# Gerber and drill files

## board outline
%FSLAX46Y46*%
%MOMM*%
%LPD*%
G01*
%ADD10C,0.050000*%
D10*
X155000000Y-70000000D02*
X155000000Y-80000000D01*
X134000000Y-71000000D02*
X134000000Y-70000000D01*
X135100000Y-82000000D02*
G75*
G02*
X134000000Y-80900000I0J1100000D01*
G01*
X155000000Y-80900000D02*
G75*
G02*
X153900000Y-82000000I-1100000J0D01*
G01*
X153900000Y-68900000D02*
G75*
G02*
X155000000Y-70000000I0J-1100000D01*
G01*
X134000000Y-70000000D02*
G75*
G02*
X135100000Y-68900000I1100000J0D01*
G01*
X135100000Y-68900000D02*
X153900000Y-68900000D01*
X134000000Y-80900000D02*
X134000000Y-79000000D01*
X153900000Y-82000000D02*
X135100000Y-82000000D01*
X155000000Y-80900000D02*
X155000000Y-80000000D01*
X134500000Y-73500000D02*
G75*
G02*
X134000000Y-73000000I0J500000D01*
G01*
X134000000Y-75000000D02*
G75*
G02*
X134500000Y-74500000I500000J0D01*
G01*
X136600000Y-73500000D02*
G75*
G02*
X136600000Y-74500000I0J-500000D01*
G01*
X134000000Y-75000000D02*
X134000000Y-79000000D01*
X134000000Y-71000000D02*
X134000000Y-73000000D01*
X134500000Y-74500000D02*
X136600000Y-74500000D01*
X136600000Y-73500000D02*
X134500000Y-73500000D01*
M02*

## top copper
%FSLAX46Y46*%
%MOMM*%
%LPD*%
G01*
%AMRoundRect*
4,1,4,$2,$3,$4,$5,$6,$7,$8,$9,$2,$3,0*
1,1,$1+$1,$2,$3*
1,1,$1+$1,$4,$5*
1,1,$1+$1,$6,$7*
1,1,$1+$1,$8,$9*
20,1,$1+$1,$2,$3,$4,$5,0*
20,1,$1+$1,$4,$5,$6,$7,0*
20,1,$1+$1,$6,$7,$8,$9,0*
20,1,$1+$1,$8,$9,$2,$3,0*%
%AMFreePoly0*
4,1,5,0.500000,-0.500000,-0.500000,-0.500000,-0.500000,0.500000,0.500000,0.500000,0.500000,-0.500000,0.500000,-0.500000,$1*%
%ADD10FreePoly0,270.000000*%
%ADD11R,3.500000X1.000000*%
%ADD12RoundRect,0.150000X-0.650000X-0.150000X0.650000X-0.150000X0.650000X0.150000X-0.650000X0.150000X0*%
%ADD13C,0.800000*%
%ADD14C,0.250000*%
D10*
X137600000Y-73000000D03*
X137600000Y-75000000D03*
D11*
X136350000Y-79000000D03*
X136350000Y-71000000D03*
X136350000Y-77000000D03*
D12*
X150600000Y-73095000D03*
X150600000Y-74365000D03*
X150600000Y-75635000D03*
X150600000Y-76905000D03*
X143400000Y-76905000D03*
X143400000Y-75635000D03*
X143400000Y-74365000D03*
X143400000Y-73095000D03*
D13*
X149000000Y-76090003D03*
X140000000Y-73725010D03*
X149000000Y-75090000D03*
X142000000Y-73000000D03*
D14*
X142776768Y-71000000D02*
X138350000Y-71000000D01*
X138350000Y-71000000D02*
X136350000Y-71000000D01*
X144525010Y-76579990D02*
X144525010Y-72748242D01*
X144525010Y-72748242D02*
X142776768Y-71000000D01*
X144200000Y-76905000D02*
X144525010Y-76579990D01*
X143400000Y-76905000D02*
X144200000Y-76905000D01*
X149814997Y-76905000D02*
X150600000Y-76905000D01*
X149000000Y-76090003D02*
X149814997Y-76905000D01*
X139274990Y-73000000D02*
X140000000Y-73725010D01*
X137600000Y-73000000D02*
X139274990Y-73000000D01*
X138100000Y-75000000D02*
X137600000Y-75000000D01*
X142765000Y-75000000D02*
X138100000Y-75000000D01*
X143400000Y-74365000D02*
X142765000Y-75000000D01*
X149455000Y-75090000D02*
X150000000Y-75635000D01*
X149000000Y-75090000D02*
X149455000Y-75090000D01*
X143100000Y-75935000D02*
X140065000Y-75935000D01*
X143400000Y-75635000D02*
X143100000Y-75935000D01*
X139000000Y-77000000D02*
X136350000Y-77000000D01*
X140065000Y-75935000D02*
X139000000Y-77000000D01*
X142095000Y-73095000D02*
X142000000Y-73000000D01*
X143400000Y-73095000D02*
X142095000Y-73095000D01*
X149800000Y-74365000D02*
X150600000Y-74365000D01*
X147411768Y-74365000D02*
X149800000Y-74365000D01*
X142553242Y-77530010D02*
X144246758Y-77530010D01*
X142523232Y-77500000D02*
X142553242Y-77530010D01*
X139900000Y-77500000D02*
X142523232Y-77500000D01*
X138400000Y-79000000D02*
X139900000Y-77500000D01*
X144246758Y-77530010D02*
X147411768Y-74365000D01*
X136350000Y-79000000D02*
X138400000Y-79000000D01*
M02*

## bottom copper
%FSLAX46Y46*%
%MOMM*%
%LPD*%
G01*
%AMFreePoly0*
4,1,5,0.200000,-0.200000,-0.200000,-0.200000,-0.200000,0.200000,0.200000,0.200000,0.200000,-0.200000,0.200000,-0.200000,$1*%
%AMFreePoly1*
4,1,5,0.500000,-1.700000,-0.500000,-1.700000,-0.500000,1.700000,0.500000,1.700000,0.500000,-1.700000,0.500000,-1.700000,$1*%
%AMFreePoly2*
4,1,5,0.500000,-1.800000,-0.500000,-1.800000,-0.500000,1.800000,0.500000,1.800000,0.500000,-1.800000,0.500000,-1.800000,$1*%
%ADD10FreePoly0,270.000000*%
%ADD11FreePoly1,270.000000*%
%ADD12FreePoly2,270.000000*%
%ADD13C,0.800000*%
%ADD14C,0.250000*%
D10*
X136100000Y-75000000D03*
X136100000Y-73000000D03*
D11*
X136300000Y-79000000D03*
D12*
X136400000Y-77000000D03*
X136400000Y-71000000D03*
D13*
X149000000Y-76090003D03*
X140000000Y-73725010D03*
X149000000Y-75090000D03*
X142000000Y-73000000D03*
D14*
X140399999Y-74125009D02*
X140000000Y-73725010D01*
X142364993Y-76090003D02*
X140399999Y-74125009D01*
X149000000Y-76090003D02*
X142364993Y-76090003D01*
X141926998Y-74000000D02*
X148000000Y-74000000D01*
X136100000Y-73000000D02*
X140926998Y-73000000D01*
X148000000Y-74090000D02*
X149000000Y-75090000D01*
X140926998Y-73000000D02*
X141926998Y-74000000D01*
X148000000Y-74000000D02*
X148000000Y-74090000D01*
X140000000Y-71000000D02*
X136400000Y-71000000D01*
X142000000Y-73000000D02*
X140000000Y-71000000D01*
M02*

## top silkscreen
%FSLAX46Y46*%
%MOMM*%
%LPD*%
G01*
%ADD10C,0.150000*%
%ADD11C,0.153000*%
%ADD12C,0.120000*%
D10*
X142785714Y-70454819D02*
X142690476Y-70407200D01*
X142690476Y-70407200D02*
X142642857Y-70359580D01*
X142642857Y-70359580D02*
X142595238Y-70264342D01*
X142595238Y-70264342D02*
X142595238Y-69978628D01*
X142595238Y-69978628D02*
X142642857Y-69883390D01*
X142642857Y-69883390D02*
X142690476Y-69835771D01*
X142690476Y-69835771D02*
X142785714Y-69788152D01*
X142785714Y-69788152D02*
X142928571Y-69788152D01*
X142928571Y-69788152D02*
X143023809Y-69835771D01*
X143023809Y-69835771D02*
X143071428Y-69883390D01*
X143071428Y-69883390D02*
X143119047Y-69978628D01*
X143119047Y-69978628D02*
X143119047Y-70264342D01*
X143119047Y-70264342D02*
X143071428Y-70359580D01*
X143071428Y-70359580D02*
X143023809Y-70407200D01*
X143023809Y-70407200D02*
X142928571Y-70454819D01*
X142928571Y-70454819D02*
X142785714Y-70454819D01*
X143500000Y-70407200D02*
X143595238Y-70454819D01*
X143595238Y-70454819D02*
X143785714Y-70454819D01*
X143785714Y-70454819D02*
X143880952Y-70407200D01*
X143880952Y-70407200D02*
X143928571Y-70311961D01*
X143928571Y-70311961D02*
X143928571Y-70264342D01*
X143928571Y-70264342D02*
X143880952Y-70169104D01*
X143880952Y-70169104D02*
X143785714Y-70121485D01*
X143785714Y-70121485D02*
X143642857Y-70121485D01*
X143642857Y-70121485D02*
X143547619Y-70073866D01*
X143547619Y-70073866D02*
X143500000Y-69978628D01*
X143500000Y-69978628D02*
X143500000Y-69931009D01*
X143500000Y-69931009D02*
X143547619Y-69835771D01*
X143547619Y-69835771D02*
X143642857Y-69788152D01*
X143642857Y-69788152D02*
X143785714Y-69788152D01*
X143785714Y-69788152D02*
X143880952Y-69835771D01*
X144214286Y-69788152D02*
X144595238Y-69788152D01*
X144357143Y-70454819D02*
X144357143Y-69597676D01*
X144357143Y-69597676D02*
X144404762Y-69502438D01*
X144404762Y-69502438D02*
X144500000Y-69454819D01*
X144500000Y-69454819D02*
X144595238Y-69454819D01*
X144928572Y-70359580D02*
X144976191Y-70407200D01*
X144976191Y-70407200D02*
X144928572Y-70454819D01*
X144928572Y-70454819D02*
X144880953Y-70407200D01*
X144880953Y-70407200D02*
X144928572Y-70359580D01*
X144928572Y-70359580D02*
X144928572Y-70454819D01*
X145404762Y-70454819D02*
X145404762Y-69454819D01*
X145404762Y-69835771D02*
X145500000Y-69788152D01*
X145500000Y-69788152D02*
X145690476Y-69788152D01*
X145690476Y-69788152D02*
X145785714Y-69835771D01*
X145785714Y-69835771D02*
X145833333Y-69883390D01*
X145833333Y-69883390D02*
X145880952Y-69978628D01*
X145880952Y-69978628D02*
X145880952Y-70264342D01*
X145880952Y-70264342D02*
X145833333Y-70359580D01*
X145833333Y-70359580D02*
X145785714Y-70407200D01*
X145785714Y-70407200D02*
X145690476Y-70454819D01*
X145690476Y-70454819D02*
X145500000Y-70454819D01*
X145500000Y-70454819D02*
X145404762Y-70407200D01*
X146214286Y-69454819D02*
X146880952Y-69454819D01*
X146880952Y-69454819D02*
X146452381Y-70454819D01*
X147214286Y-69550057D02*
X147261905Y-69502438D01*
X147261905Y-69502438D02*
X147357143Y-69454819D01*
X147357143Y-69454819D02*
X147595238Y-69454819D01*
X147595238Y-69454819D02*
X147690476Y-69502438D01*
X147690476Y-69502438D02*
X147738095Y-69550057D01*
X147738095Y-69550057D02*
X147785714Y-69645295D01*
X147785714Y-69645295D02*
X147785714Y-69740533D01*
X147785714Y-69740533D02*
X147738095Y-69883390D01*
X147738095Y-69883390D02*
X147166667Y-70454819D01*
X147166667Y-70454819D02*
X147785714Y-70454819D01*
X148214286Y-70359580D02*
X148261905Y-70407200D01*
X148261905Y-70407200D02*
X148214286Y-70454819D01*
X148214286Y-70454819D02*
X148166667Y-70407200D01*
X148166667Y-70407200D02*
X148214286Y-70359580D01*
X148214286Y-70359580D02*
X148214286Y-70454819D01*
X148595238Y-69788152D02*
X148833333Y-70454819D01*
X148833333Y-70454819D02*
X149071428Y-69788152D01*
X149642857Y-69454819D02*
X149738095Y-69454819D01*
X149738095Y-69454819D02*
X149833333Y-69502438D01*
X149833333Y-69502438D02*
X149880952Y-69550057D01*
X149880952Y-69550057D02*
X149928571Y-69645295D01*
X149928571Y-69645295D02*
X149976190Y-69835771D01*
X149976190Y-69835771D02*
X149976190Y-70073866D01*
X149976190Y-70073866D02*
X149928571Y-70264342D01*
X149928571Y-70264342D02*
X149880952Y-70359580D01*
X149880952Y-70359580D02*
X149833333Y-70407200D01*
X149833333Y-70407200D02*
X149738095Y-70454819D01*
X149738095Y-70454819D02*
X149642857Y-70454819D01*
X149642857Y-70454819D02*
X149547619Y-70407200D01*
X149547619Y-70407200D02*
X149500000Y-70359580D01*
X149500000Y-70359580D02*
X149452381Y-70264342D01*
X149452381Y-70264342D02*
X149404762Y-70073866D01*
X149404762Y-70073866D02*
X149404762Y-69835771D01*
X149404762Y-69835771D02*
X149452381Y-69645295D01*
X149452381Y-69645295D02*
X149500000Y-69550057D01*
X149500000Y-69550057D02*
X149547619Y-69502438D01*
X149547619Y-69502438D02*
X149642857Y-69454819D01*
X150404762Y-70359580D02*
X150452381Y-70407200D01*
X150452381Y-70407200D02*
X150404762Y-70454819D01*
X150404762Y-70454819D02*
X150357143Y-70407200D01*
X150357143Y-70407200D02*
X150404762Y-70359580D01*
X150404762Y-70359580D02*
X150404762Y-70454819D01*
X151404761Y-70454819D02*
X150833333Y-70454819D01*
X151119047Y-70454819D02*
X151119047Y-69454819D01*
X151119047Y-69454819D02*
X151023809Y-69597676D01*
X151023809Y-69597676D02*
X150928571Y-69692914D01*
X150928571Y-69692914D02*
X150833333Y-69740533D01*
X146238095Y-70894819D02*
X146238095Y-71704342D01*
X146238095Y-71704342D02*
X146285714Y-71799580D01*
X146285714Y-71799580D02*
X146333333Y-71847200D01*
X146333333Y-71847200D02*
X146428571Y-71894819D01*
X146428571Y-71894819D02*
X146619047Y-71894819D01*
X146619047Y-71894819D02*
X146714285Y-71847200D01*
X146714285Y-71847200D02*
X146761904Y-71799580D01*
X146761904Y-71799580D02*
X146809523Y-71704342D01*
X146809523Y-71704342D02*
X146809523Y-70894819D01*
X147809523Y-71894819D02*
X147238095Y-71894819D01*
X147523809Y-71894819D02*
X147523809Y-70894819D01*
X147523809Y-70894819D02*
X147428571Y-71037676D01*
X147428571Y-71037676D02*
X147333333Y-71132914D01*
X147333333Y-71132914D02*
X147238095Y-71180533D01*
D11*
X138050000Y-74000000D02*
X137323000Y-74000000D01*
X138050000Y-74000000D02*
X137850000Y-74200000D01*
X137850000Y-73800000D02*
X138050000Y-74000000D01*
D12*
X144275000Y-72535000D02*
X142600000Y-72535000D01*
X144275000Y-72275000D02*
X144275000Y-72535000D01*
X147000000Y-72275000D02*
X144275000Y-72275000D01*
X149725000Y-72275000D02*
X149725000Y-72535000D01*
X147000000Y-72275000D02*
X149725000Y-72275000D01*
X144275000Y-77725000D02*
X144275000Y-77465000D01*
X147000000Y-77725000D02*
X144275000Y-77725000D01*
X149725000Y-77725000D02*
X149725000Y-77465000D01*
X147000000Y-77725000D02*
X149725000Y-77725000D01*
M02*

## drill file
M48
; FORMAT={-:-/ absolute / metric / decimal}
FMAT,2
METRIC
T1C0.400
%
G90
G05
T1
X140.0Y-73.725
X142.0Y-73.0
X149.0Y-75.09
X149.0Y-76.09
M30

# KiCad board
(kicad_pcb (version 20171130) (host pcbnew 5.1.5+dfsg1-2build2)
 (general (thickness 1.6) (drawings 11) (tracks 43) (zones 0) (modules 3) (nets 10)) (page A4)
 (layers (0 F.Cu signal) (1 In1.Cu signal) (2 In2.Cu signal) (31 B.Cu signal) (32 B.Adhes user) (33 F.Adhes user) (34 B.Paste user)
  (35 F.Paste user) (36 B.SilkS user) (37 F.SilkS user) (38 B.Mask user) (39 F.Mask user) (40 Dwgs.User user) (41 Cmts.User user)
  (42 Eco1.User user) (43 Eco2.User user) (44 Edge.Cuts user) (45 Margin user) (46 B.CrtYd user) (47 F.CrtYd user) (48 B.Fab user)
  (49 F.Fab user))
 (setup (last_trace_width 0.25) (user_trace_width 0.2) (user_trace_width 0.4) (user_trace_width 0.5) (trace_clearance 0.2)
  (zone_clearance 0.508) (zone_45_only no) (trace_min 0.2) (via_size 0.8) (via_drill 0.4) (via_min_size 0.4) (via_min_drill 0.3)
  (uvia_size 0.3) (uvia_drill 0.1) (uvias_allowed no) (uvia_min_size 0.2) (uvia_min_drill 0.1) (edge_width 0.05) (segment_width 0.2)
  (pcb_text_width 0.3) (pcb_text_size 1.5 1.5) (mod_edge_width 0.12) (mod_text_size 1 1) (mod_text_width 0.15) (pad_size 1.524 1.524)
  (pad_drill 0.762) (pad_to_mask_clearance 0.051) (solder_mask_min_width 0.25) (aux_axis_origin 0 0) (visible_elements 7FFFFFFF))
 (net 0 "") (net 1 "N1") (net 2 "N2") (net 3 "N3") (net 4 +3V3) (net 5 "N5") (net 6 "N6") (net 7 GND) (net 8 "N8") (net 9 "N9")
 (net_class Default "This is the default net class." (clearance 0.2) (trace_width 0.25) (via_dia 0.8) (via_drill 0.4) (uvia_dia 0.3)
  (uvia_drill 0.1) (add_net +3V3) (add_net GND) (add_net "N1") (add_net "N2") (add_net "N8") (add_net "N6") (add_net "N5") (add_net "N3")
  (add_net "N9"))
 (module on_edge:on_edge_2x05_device (layer F.Cu) (at 134 75 270)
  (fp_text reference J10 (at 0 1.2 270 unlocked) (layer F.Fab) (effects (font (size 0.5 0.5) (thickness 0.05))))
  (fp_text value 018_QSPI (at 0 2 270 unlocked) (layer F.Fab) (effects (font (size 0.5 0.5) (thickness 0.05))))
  (fp_arc (start -2 -0.5) (end -2 0) (angle -90) (layer Edge.Cuts) (width 0.05))
  (fp_arc (start 0 -0.5) (end -0.5 -0.5) (angle -90) (layer Edge.Cuts) (width 0.05))
  (fp_arc (start -1 -2.6) (end -0.5 -2.6) (angle -180) (layer Edge.Cuts) (width 0.05))
  (fp_line (start 0 0) (end 4 0) (layer Edge.Cuts) (width 0.05))
  (fp_line (start -4 0) (end -2 0) (layer Edge.Cuts) (width 0.05))
  (fp_line (start -1 -4.05) (end -1 -3.323) (layer F.SilkS) (width 0.153))
  (fp_line (start -1 -4.05) (end -0.8 -3.85) (layer F.SilkS) (width 0.153))
  (fp_line (start -1.2 -3.85) (end -1 -4.05) (layer F.SilkS) (width 0.153))
  (fp_line (start -0.5 -0.5) (end -0.5 -2.6) (layer Edge.Cuts) (width 0.05))
  (fp_line (start -1.5 -2.6) (end -1.5 -0.5) (layer Edge.Cuts) (width 0.05))
  (pad 2 smd custom (at -2 -3.6 270) (size 1 1) (layers F.Cu F.Mask) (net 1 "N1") (zone_connect 0)
   (options (clearance outline) (anchor rect)) (primitives))
  (pad 3 smd custom (at 0 -3.6 270) (size 1 1) (layers F.Cu F.Mask) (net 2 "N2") (zone_connect 0)
   (options (clearance outline) (anchor rect)) (primitives))
  (pad 8 smd custom (at 0 -2.1 270) (size 0.4 0.4) (layers B.Cu B.Mask) (zone_connect 0) (options (clearance outline) (anchor rect))
   (primitives))
  (pad 7 smd custom (at -2 -2.1 270) (size 0.4 0.4) (layers B.Cu B.Mask) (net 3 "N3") (zone_connect 0)
   (options (clearance outline) (anchor rect)) (primitives))
  (pad 10 smd custom (at 4 -2.3 270) (size 1 3.4) (layers B.Cu B.Mask) (zone_connect 0) (options (clearance outline) (anchor rect))
   (primitives))
  (pad 9 smd custom (at 2 -2.4 270) (size 1 3.6) (layers B.Cu B.Mask) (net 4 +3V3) (zone_connect 0)
   (options (clearance outline) (anchor rect)) (primitives))
  (pad 6 smd custom (at -4 -2.4 270) (size 1 3.6) (layers B.Cu B.Mask) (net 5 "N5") (zone_connect 0)
   (options (clearance outline) (anchor rect)) (primitives))
  (pad 5 smd rect (at 4 -2.35 90) (size 1 3.5) (layers F.Cu F.Mask) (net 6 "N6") (zone_connect 0))
  (pad 1 smd rect (at -4 -2.35 90) (size 1 3.5) (layers F.Cu F.Mask) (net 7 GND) (zone_connect 0))
  (pad 4 smd rect (at 2 -2.35 90) (size 1 3.5) (layers F.Cu F.Mask) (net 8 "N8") (zone_connect 0)))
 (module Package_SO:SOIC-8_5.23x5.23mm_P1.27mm (layer F.Cu) (at 147 75)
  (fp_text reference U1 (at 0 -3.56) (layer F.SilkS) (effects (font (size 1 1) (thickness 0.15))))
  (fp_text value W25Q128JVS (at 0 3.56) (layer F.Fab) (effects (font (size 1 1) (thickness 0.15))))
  (fp_line (start -2.725 -2.465) (end -4.4 -2.465) (layer F.SilkS) (width 0.12))
  (fp_line (start -2.725 -2.725) (end -2.725 -2.465) (layer F.SilkS) (width 0.12))
  (fp_line (start 0 -2.725) (end -2.725 -2.725) (layer F.SilkS) (width 0.12))
  (fp_line (start 2.725 -2.725) (end 2.725 -2.465) (layer F.SilkS) (width 0.12))
  (fp_line (start 0 -2.725) (end 2.725 -2.725) (layer F.SilkS) (width 0.12))
  (fp_line (start -2.725 2.725) (end -2.725 2.465) (layer F.SilkS) (width 0.12))
  (fp_line (start 0 2.725) (end -2.725 2.725) (layer F.SilkS) (width 0.12))
  (fp_line (start 2.725 2.725) (end 2.725 2.465) (layer F.SilkS) (width 0.12))
  (fp_line (start 0 2.725) (end 2.725 2.725) (layer F.SilkS) (width 0.12))
  (pad 8 smd roundrect (at 3.6 -1.905) (size 1.6 0.6) (layers F.Cu F.Paste F.Mask) (roundrect_rratio 0.25) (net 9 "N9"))
  (pad 7 smd roundrect (at 3.6 -0.635) (size 1.6 0.6) (layers F.Cu F.Paste F.Mask) (roundrect_rratio 0.25) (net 6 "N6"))
  (pad 6 smd roundrect (at 3.6 0.635) (size 1.6 0.6) (layers F.Cu F.Paste F.Mask) (roundrect_rratio 0.25) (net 3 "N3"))
  (pad 5 smd roundrect (at 3.6 1.905) (size 1.6 0.6) (layers F.Cu F.Paste F.Mask) (roundrect_rratio 0.25) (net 1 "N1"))
  (pad 4 smd roundrect (at -3.6 1.905) (size 1.6 0.6) (layers F.Cu F.Paste F.Mask) (roundrect_rratio 0.25) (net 7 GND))
  (pad 3 smd roundrect (at -3.6 0.635) (size 1.6 0.6) (layers F.Cu F.Paste F.Mask) (roundrect_rratio 0.25) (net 8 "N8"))
  (pad 2 smd roundrect (at -3.6 -0.635) (size 1.6 0.6) (layers F.Cu F.Paste F.Mask) (roundrect_rratio 0.25) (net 2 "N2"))
  (pad 1 smd roundrect (at -3.6 -1.905) (size 1.6 0.6) (layers F.Cu F.Paste F.Mask) (roundrect_rratio 0.25) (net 5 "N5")))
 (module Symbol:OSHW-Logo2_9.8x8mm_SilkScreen (layer B.Cu) (at 146 78 180)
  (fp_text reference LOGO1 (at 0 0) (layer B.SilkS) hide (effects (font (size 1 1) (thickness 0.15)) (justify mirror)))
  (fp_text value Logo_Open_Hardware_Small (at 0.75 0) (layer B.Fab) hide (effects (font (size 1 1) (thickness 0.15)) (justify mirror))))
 (gr_line (start 155 70) (end 155 80) (layer Edge.Cuts) (width 0.05))
 (gr_line (start 134 71) (end 134 70) (layer Edge.Cuts) (width 0.05))
 (gr_arc (start 135.1 80.9) (end 134 80.9) (angle -90) (layer Edge.Cuts) (width 0.05))
 (gr_arc (start 153.9 80.9) (end 153.9 82) (angle -90) (layer Edge.Cuts) (width 0.05))
 (gr_arc (start 153.9 70) (end 155 70) (angle -90) (layer Edge.Cuts) (width 0.05))
 (gr_arc (start 135.1 70) (end 135.1 68.9) (angle -90) (layer Edge.Cuts) (width 0.05))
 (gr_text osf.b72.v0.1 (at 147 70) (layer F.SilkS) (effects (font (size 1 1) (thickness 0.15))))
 (gr_line (start 135.1 68.9) (end 153.9 68.9) (layer Edge.Cuts) (width 0.05))
 (gr_line (start 134 80.9) (end 134 79) (layer Edge.Cuts) (width 0.05))
 (gr_line (start 153.9 82) (end 135.1 82) (layer Edge.Cuts) (width 0.05))
 (gr_line (start 155 80.9) (end 155 80) (layer Edge.Cuts) (width 0.05))
 (segment (start 142.776768 71) (end 138.35 71) (width 0.25) (layer F.Cu) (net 7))
 (segment (start 138.35 71) (end 136.35 71) (width 0.25) (layer F.Cu) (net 7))
 (segment (start 144.52501 76.57999) (end 144.52501 72.748242) (width 0.25) (layer F.Cu) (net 7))
 (segment (start 144.52501 72.748242) (end 142.776768 71) (width 0.25) (layer F.Cu) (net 7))
 (segment (start 144.2 76.905) (end 144.52501 76.57999) (width 0.25) (layer F.Cu) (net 7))
 (segment (start 143.4 76.905) (end 144.2 76.905) (width 0.25) (layer F.Cu) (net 7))
 (via (at 149 76.090003) (size 0.8) (drill 0.4) (layers F.Cu B.Cu) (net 1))
 (segment (start 149.814997 76.905) (end 150.6 76.905) (width 0.25) (layer F.Cu) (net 1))
 (segment (start 149 76.090003) (end 149.814997 76.905) (width 0.25) (layer F.Cu) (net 1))
 (segment (start 140.399999 74.125009) (end 140 73.72501) (width 0.25) (layer B.Cu) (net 1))
 (segment (start 142.364993 76.090003) (end 140.399999 74.125009) (width 0.25) (layer B.Cu) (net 1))
 (segment (start 139.27499 73) (end 140 73.72501) (width 0.25) (layer F.Cu) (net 1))
 (segment (start 137.6 73) (end 139.27499 73) (width 0.25) (layer F.Cu) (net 1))
 (via (at 140 73.72501) (size 0.8) (drill 0.4) (layers F.Cu B.Cu) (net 1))
 (segment (start 149 76.090003) (end 142.364993 76.090003) (width 0.25) (layer B.Cu) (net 1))
 (segment (start 138.1 75) (end 137.6 75) (width 0.25) (layer F.Cu) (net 2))
 (segment (start 142.765 75) (end 138.1 75) (width 0.25) (layer F.Cu) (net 2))
 (segment (start 143.4 74.365) (end 142.765 75) (width 0.25) (layer F.Cu) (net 2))
 (via (at 149 75.09) (size 0.8) (drill 0.4) (layers F.Cu B.Cu) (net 3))
 (segment (start 149.455 75.09) (end 150 75.635) (width 0.25) (layer F.Cu) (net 3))
 (segment (start 149 75.09) (end 149.455 75.09) (width 0.25) (layer F.Cu) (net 3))
 (segment (start 141.926998 74) (end 148 74) (width 0.25) (layer B.Cu) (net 3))
 (segment (start 136.1 73) (end 140.926998 73) (width 0.25) (layer B.Cu) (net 3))
 (segment (start 148 74.09) (end 149 75.09) (width 0.25) (layer B.Cu) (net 3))
 (segment (start 140.926998 73) (end 141.926998 74) (width 0.25) (layer B.Cu) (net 3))
 (segment (start 148 74) (end 148 74.09) (width 0.25) (layer B.Cu) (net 3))
 (segment (start 143.1 75.935) (end 140.065 75.935) (width 0.25) (layer F.Cu) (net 8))
 (segment (start 143.4 75.635) (end 143.1 75.935) (width 0.25) (layer F.Cu) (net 8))
 (segment (start 139 77) (end 136.35 77) (width 0.25) (layer F.Cu) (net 8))
 (segment (start 140.065 75.935) (end 139 77) (width 0.25) (layer F.Cu) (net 8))
 (via (at 142 73) (size 0.8) (drill 0.4) (layers F.Cu B.Cu) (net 5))
 (segment (start 142.095 73.095) (end 142 73) (width 0.25) (layer F.Cu) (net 5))
 (segment (start 143.4 73.095) (end 142.095 73.095) (width 0.25) (layer F.Cu) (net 5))
 (segment (start 140 71) (end 136.4 71) (width 0.25) (layer B.Cu) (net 5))
 (segment (start 142 73) (end 140 71) (width 0.25) (layer B.Cu) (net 5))
 (segment (start 149.8 74.365) (end 150.6 74.365) (width 0.25) (layer F.Cu) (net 6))
 (segment (start 147.411768 74.365) (end 149.8 74.365) (width 0.25) (layer F.Cu) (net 6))
 (segment (start 142.553242 77.53001) (end 144.246758 77.53001) (width 0.25) (layer F.Cu) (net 6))
 (segment (start 142.523232 77.5) (end 142.553242 77.53001) (width 0.25) (layer F.Cu) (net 6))
 (segment (start 139.9 77.5) (end 142.523232 77.5) (width 0.25) (layer F.Cu) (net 6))
 (segment (start 138.4 79) (end 139.9 77.5) (width 0.25) (layer F.Cu) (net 6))
 (segment (start 144.246758 77.53001) (end 147.411768 74.365) (width 0.25) (layer F.Cu) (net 6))
 (segment (start 136.35 79) (end 138.4 79) (width 0.25) (layer F.Cu) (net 6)))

